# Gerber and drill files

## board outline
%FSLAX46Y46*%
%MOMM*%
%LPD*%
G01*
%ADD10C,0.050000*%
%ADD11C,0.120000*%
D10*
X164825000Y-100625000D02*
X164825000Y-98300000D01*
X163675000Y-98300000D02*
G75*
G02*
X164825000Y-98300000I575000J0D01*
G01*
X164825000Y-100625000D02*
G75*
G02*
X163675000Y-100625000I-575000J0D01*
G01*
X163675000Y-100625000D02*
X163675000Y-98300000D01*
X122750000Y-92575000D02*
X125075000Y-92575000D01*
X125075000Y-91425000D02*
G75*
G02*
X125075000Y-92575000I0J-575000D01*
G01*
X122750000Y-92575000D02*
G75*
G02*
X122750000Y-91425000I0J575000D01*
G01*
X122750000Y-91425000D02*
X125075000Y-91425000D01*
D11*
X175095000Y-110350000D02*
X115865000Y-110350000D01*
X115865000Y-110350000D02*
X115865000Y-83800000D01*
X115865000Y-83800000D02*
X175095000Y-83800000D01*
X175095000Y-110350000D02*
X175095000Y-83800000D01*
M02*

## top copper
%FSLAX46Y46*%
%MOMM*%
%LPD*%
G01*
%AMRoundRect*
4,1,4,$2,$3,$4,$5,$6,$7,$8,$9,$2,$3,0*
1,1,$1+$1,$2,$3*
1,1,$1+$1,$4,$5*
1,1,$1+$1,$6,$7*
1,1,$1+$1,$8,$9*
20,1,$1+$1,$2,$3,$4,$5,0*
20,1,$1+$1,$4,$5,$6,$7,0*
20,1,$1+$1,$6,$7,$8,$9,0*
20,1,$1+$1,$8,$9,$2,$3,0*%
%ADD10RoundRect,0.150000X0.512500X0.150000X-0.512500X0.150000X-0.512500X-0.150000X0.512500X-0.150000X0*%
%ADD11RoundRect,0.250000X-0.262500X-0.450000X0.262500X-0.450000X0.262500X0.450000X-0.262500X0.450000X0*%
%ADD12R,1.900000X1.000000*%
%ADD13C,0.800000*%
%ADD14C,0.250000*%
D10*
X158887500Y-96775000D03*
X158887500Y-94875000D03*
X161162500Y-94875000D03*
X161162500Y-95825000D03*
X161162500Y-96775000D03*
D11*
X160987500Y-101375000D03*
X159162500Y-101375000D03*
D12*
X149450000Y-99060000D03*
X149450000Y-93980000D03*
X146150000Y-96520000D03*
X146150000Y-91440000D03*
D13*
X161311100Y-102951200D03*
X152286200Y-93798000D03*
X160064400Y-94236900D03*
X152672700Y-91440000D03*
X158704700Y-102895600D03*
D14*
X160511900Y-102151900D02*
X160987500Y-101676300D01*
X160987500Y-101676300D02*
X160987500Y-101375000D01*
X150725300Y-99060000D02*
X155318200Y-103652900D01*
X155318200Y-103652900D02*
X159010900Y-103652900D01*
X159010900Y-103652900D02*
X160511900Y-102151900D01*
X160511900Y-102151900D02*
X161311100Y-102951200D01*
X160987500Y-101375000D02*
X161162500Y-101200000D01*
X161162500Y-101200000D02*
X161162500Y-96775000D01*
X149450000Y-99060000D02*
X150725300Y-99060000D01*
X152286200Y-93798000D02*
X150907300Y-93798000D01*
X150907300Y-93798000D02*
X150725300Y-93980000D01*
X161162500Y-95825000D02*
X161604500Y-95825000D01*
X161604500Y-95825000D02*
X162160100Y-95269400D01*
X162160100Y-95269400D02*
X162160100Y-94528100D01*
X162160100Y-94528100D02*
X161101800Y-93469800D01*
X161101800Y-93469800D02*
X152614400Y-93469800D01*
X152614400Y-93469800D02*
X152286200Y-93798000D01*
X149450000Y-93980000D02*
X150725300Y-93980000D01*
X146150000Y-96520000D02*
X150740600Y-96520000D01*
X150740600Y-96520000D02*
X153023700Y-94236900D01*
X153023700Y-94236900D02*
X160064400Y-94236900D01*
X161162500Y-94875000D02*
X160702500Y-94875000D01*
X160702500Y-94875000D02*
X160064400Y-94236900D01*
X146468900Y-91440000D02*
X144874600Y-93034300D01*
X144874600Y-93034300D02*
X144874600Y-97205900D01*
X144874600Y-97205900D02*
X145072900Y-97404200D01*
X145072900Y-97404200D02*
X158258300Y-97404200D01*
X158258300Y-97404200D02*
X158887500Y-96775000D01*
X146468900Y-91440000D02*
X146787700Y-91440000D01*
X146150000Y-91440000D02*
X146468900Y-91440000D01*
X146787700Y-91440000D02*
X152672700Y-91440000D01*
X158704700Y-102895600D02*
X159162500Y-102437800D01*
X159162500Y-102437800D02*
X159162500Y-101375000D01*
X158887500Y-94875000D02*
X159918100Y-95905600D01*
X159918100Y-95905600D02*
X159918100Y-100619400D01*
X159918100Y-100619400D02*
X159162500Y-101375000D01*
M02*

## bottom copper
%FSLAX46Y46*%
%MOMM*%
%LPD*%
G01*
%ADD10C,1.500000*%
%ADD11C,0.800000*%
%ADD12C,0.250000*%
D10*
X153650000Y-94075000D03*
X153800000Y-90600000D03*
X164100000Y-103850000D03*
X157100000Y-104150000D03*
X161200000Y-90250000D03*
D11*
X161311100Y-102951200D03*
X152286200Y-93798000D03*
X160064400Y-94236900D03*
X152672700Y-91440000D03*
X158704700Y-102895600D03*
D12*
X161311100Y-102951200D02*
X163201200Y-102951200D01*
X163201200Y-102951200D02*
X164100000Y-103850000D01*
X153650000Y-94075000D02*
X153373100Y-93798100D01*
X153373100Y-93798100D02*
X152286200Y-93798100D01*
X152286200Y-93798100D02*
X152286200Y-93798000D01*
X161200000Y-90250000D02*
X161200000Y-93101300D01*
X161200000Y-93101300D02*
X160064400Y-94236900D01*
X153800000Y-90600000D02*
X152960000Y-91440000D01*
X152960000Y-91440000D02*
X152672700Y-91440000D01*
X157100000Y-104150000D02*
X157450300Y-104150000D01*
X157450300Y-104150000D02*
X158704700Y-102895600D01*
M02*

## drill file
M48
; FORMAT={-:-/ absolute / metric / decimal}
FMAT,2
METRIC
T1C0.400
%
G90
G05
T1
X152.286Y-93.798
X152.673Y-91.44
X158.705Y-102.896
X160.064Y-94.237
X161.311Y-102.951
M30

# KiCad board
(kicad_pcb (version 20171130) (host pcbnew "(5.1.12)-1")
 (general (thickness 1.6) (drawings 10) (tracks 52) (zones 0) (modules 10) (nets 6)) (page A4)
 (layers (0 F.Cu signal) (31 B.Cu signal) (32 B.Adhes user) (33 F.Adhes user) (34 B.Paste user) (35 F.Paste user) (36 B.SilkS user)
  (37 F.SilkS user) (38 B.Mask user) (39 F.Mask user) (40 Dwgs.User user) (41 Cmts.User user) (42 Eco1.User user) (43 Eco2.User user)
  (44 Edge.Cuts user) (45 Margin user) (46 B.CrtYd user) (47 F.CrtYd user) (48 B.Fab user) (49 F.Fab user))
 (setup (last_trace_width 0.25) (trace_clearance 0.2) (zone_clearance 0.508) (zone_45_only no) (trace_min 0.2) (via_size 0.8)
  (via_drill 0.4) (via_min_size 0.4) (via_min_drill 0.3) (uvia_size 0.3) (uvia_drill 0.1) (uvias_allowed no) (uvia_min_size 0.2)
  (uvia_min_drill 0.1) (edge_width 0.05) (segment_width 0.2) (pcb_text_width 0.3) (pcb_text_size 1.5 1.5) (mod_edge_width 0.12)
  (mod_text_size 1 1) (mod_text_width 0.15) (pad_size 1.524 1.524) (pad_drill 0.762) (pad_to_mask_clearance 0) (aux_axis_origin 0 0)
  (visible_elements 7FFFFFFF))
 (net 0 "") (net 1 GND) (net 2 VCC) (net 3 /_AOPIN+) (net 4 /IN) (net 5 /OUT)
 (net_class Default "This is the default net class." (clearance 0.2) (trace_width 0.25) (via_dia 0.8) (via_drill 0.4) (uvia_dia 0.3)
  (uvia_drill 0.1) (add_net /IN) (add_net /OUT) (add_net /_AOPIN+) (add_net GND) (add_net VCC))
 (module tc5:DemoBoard (layer F.Cu) (at 127.325 91.1)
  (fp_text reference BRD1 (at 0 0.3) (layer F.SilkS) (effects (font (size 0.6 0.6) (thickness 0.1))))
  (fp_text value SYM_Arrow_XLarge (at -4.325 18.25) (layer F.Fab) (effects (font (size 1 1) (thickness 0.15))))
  (fp_line (start 47.77 19.25) (end -11.46 19.25) (layer Edge.Cuts) (width 0.12))
  (fp_line (start -11.46 19.25) (end -11.46 -7.3) (layer Edge.Cuts) (width 0.12))
  (fp_line (start -11.46 -7.3) (end 47.77 -7.3) (layer Edge.Cuts) (width 0.12))
  (fp_line (start 47.77 19.25) (end 47.77 -7.3) (layer Edge.Cuts) (width 0.12)))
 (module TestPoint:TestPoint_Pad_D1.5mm (layer B.Cu) (at 153.65 94.075)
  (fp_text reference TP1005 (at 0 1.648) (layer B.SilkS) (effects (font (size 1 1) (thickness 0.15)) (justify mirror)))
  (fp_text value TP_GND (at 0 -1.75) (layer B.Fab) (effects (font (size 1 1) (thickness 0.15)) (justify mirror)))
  (pad 1 smd circle (at 0 0) (size 1.5 1.5) (layers B.Cu B.Mask) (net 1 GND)))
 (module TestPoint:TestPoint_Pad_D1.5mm (layer B.Cu) (at 153.8 90.6)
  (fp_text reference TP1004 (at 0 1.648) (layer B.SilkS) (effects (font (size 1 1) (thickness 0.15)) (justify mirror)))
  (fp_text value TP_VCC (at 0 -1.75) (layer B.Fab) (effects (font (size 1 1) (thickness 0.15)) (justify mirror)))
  (pad 1 smd circle (at 0 0) (size 1.5 1.5) (layers B.Cu B.Mask) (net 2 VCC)))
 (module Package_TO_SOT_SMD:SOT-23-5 (layer F.Cu) (at 160.025 95.825 180)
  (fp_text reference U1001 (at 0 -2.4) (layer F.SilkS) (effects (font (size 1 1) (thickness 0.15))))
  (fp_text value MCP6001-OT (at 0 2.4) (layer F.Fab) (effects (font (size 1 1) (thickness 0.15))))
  (pad 5 smd roundrect (at 1.1375 -0.95 180) (size 1.325 0.6) (layers F.Cu F.Paste F.Mask) (roundrect_rratio 0.25) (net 2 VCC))
  (pad 4 smd roundrect (at 1.1375 0.95 180) (size 1.325 0.6) (layers F.Cu F.Paste F.Mask) (roundrect_rratio 0.25) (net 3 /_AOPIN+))
  (pad 3 smd roundrect (at -1.1375 0.95 180) (size 1.325 0.6) (layers F.Cu F.Paste F.Mask) (roundrect_rratio 0.25) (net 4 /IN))
  (pad 2 smd roundrect (at -1.1375 0 180) (size 1.325 0.6) (layers F.Cu F.Paste F.Mask) (roundrect_rratio 0.25) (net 1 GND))
  (pad 1 smd roundrect (at -1.1375 -0.95 180) (size 1.325 0.6) (layers F.Cu F.Paste F.Mask) (roundrect_rratio 0.25) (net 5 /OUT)))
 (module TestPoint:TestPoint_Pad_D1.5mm (layer B.Cu) (at 164.1 103.85 180)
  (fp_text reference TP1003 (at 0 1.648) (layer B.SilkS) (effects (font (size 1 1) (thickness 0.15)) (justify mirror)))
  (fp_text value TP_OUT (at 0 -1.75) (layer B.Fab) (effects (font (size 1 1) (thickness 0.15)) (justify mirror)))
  (pad 1 smd circle (at 0 0 180) (size 1.5 1.5) (layers B.Cu B.Mask) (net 5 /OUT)))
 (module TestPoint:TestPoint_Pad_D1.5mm (layer B.Cu) (at 157.1 104.15)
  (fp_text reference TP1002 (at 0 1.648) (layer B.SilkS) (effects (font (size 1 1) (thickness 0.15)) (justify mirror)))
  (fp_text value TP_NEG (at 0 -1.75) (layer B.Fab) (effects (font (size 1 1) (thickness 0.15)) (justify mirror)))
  (pad 1 smd circle (at 0 0) (size 1.5 1.5) (layers B.Cu B.Mask) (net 3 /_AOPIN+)))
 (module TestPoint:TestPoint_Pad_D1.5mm (layer B.Cu) (at 161.2 90.25)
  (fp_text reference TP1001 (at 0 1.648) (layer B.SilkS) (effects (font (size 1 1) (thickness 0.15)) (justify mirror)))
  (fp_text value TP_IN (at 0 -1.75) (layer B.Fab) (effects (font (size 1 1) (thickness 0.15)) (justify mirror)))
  (pad 1 smd circle (at 0 0) (size 1.5 1.5) (layers B.Cu B.Mask) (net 4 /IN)))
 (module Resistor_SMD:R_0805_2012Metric (layer F.Cu) (at 160.075 101.375)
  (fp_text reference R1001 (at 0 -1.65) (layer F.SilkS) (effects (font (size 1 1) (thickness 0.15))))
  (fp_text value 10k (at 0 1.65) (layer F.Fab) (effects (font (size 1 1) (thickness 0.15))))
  (pad 2 smd roundrect (at 0.9125 0) (size 1.025 1.4) (layers F.Cu F.Paste F.Mask) (roundrect_rratio 0.243902) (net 5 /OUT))
  (pad 1 smd roundrect (at -0.9125 0) (size 1.025 1.4) (layers F.Cu F.Paste F.Mask) (roundrect_rratio 0.243902) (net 3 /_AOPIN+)))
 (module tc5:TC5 (layer F.Cu) (at 135.3 97.9)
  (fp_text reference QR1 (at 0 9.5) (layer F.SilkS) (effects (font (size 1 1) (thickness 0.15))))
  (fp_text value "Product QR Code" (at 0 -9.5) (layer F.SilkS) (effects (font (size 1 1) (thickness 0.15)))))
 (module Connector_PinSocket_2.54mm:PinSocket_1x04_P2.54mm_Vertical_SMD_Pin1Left (layer F.Cu) (at 147.8 95.25)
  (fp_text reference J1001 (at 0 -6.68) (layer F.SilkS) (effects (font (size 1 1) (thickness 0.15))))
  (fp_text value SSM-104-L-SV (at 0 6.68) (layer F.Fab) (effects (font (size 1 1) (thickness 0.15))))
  (pad 4 smd rect (at 1.65 3.81) (size 1.9 1) (layers F.Cu F.Paste F.Mask) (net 5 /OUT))
  (pad 2 smd rect (at 1.65 -1.27) (size 1.9 1) (layers F.Cu F.Paste F.Mask) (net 1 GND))
  (pad 3 smd rect (at -1.65 1.27) (size 1.9 1) (layers F.Cu F.Paste F.Mask) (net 4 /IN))
  (pad 1 smd rect (at -1.65 -3.81) (size 1.9 1) (layers F.Cu F.Paste F.Mask) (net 2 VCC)))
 (gr_line (start 164.825 100.625) (end 164.825 98.3) (layer Edge.Cuts) (width 0.05))
 (gr_arc (start 164.25 98.3) (end 164.825 98.3) (angle -180) (layer Edge.Cuts) (width 0.05))
 (gr_arc (start 164.25 100.625) (end 163.675 100.625) (angle -180) (layer Edge.Cuts) (width 0.05))
 (gr_line (start 163.675 100.625) (end 163.675 98.3) (layer Edge.Cuts) (width 0.05))
 (gr_line (start 122.75 92.575) (end 125.075 92.575) (layer Edge.Cuts) (width 0.05))
 (gr_arc (start 125.075 92) (end 125.075 92.575) (angle -180) (layer Edge.Cuts) (width 0.05))
 (gr_arc (start 122.75 92) (end 122.75 91.425) (angle -180) (layer Edge.Cuts) (width 0.05))
 (gr_line (start 122.75 91.425) (end 125.075 91.425) (layer Edge.Cuts) (width 0.05))
 (segment (start 160.5119 102.1519) (end 160.9875 101.6763) (width 0.25) (layer F.Cu) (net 5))
 (segment (start 160.9875 101.6763) (end 160.9875 101.375) (width 0.25) (layer F.Cu) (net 5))
 (segment (start 150.7253 99.06) (end 155.3182 103.6529) (width 0.25) (layer F.Cu) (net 5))
 (segment (start 155.3182 103.6529) (end 159.0109 103.6529) (width 0.25) (layer F.Cu) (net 5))
 (segment (start 159.0109 103.6529) (end 160.5119 102.1519) (width 0.25) (layer F.Cu) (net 5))
 (segment (start 160.5119 102.1519) (end 161.3111 102.9512) (width 0.25) (layer F.Cu) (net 5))
 (segment (start 161.3111 102.9512) (end 163.2012 102.9512) (width 0.25) (layer B.Cu) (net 5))
 (segment (start 163.2012 102.9512) (end 164.1 103.85) (width 0.25) (layer B.Cu) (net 5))
 (segment (start 160.9875 101.375) (end 161.1625 101.2) (width 0.25) (layer F.Cu) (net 5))
 (segment (start 161.1625 101.2) (end 161.1625 96.775) (width 0.25) (layer F.Cu) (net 5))
 (segment (start 149.45 99.06) (end 150.7253 99.06) (width 0.25) (layer F.Cu) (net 5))
 (via (at 161.3111 102.9512) (size 0.8) (layers F.Cu B.Cu) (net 5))
 (segment (start 152.2862 93.798) (end 150.9073 93.798) (width 0.25) (layer F.Cu) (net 1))
 (segment (start 150.9073 93.798) (end 150.7253 93.98) (width 0.25) (layer F.Cu) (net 1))
 (segment (start 161.1625 95.825) (end 161.6045 95.825) (width 0.25) (layer F.Cu) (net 1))
 (segment (start 161.6045 95.825) (end 162.1601 95.2694) (width 0.25) (layer F.Cu) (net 1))
 (segment (start 162.1601 95.2694) (end 162.1601 94.5281) (width 0.25) (layer F.Cu) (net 1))
 (segment (start 162.1601 94.5281) (end 161.1018 93.4698) (width 0.25) (layer F.Cu) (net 1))
 (segment (start 161.1018 93.4698) (end 152.6144 93.4698) (width 0.25) (layer F.Cu) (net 1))
 (segment (start 152.6144 93.4698) (end 152.2862 93.798) (width 0.25) (layer F.Cu) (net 1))
 (segment (start 153.65 94.075) (end 153.3731 93.7981) (width 0.25) (layer B.Cu) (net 1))
 (segment (start 153.3731 93.7981) (end 152.2862 93.7981) (width 0.25) (layer B.Cu) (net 1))
 (segment (start 152.2862 93.7981) (end 152.2862 93.798) (width 0.25) (layer B.Cu) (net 1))
 (segment (start 149.45 93.98) (end 150.7253 93.98) (width 0.25) (layer F.Cu) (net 1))
 (via (at 152.2862 93.798) (size 0.8) (layers F.Cu B.Cu) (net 1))
 (segment (start 146.15 96.52) (end 150.7406 96.52) (width 0.25) (layer F.Cu) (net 4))
 (segment (start 150.7406 96.52) (end 153.0237 94.2369) (width 0.25) (layer F.Cu) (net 4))
 (segment (start 153.0237 94.2369) (end 160.0644 94.2369) (width 0.25) (layer F.Cu) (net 4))
 (segment (start 161.1625 94.875) (end 160.7025 94.875) (width 0.25) (layer F.Cu) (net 4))
 (segment (start 160.7025 94.875) (end 160.0644 94.2369) (width 0.25) (layer F.Cu) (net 4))
 (segment (start 161.2 90.25) (end 161.2 93.1013) (width 0.25) (layer B.Cu) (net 4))
 (segment (start 161.2 93.1013) (end 160.0644 94.2369) (width 0.25) (layer B.Cu) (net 4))
 (via (at 160.0644 94.2369) (size 0.8) (layers F.Cu B.Cu) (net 4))
 (segment (start 146.4689 91.44) (end 144.8746 93.0343) (width 0.25) (layer F.Cu) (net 2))
 (segment (start 144.8746 93.0343) (end 144.8746 97.2059) (width 0.25) (layer F.Cu) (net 2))
 (segment (start 144.8746 97.2059) (end 145.0729 97.4042) (width 0.25) (layer F.Cu) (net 2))
 (segment (start 145.0729 97.4042) (end 158.2583 97.4042) (width 0.25) (layer F.Cu) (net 2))
 (segment (start 158.2583 97.4042) (end 158.8875 96.775) (width 0.25) (layer F.Cu) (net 2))
 (segment (start 146.4689 91.44) (end 146.7877 91.44) (width 0.25) (layer F.Cu) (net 2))
 (segment (start 146.15 91.44) (end 146.4689 91.44) (width 0.25) (layer F.Cu) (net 2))
 (segment (start 146.7877 91.44) (end 152.6727 91.44) (width 0.25) (layer F.Cu) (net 2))
 (segment (start 153.8 90.6) (end 152.96 91.44) (width 0.25) (layer B.Cu) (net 2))
 (segment (start 152.96 91.44) (end 152.6727 91.44) (width 0.25) (layer B.Cu) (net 2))
 (via (at 152.6727 91.44) (size 0.8) (layers F.Cu B.Cu) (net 2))
 (segment (start 158.7047 102.8956) (end 159.1625 102.4378) (width 0.25) (layer F.Cu) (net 3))
 (segment (start 159.1625 102.4378) (end 159.1625 101.375) (width 0.25) (layer F.Cu) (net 3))
 (segment (start 157.1 104.15) (end 157.4503 104.15) (width 0.25) (layer B.Cu) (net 3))
 (segment (start 157.4503 104.15) (end 158.7047 102.8956) (width 0.25) (layer B.Cu) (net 3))
 (segment (start 158.8875 94.875) (end 159.9181 95.9056) (width 0.25) (layer F.Cu) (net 3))
 (segment (start 159.9181 95.9056) (end 159.9181 100.6194) (width 0.25) (layer F.Cu) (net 3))
 (segment (start 159.9181 100.6194) (end 159.1625 101.375) (width 0.25) (layer F.Cu) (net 3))
 (via (at 158.7047 102.8956) (size 0.8) (layers F.Cu B.Cu) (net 3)))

